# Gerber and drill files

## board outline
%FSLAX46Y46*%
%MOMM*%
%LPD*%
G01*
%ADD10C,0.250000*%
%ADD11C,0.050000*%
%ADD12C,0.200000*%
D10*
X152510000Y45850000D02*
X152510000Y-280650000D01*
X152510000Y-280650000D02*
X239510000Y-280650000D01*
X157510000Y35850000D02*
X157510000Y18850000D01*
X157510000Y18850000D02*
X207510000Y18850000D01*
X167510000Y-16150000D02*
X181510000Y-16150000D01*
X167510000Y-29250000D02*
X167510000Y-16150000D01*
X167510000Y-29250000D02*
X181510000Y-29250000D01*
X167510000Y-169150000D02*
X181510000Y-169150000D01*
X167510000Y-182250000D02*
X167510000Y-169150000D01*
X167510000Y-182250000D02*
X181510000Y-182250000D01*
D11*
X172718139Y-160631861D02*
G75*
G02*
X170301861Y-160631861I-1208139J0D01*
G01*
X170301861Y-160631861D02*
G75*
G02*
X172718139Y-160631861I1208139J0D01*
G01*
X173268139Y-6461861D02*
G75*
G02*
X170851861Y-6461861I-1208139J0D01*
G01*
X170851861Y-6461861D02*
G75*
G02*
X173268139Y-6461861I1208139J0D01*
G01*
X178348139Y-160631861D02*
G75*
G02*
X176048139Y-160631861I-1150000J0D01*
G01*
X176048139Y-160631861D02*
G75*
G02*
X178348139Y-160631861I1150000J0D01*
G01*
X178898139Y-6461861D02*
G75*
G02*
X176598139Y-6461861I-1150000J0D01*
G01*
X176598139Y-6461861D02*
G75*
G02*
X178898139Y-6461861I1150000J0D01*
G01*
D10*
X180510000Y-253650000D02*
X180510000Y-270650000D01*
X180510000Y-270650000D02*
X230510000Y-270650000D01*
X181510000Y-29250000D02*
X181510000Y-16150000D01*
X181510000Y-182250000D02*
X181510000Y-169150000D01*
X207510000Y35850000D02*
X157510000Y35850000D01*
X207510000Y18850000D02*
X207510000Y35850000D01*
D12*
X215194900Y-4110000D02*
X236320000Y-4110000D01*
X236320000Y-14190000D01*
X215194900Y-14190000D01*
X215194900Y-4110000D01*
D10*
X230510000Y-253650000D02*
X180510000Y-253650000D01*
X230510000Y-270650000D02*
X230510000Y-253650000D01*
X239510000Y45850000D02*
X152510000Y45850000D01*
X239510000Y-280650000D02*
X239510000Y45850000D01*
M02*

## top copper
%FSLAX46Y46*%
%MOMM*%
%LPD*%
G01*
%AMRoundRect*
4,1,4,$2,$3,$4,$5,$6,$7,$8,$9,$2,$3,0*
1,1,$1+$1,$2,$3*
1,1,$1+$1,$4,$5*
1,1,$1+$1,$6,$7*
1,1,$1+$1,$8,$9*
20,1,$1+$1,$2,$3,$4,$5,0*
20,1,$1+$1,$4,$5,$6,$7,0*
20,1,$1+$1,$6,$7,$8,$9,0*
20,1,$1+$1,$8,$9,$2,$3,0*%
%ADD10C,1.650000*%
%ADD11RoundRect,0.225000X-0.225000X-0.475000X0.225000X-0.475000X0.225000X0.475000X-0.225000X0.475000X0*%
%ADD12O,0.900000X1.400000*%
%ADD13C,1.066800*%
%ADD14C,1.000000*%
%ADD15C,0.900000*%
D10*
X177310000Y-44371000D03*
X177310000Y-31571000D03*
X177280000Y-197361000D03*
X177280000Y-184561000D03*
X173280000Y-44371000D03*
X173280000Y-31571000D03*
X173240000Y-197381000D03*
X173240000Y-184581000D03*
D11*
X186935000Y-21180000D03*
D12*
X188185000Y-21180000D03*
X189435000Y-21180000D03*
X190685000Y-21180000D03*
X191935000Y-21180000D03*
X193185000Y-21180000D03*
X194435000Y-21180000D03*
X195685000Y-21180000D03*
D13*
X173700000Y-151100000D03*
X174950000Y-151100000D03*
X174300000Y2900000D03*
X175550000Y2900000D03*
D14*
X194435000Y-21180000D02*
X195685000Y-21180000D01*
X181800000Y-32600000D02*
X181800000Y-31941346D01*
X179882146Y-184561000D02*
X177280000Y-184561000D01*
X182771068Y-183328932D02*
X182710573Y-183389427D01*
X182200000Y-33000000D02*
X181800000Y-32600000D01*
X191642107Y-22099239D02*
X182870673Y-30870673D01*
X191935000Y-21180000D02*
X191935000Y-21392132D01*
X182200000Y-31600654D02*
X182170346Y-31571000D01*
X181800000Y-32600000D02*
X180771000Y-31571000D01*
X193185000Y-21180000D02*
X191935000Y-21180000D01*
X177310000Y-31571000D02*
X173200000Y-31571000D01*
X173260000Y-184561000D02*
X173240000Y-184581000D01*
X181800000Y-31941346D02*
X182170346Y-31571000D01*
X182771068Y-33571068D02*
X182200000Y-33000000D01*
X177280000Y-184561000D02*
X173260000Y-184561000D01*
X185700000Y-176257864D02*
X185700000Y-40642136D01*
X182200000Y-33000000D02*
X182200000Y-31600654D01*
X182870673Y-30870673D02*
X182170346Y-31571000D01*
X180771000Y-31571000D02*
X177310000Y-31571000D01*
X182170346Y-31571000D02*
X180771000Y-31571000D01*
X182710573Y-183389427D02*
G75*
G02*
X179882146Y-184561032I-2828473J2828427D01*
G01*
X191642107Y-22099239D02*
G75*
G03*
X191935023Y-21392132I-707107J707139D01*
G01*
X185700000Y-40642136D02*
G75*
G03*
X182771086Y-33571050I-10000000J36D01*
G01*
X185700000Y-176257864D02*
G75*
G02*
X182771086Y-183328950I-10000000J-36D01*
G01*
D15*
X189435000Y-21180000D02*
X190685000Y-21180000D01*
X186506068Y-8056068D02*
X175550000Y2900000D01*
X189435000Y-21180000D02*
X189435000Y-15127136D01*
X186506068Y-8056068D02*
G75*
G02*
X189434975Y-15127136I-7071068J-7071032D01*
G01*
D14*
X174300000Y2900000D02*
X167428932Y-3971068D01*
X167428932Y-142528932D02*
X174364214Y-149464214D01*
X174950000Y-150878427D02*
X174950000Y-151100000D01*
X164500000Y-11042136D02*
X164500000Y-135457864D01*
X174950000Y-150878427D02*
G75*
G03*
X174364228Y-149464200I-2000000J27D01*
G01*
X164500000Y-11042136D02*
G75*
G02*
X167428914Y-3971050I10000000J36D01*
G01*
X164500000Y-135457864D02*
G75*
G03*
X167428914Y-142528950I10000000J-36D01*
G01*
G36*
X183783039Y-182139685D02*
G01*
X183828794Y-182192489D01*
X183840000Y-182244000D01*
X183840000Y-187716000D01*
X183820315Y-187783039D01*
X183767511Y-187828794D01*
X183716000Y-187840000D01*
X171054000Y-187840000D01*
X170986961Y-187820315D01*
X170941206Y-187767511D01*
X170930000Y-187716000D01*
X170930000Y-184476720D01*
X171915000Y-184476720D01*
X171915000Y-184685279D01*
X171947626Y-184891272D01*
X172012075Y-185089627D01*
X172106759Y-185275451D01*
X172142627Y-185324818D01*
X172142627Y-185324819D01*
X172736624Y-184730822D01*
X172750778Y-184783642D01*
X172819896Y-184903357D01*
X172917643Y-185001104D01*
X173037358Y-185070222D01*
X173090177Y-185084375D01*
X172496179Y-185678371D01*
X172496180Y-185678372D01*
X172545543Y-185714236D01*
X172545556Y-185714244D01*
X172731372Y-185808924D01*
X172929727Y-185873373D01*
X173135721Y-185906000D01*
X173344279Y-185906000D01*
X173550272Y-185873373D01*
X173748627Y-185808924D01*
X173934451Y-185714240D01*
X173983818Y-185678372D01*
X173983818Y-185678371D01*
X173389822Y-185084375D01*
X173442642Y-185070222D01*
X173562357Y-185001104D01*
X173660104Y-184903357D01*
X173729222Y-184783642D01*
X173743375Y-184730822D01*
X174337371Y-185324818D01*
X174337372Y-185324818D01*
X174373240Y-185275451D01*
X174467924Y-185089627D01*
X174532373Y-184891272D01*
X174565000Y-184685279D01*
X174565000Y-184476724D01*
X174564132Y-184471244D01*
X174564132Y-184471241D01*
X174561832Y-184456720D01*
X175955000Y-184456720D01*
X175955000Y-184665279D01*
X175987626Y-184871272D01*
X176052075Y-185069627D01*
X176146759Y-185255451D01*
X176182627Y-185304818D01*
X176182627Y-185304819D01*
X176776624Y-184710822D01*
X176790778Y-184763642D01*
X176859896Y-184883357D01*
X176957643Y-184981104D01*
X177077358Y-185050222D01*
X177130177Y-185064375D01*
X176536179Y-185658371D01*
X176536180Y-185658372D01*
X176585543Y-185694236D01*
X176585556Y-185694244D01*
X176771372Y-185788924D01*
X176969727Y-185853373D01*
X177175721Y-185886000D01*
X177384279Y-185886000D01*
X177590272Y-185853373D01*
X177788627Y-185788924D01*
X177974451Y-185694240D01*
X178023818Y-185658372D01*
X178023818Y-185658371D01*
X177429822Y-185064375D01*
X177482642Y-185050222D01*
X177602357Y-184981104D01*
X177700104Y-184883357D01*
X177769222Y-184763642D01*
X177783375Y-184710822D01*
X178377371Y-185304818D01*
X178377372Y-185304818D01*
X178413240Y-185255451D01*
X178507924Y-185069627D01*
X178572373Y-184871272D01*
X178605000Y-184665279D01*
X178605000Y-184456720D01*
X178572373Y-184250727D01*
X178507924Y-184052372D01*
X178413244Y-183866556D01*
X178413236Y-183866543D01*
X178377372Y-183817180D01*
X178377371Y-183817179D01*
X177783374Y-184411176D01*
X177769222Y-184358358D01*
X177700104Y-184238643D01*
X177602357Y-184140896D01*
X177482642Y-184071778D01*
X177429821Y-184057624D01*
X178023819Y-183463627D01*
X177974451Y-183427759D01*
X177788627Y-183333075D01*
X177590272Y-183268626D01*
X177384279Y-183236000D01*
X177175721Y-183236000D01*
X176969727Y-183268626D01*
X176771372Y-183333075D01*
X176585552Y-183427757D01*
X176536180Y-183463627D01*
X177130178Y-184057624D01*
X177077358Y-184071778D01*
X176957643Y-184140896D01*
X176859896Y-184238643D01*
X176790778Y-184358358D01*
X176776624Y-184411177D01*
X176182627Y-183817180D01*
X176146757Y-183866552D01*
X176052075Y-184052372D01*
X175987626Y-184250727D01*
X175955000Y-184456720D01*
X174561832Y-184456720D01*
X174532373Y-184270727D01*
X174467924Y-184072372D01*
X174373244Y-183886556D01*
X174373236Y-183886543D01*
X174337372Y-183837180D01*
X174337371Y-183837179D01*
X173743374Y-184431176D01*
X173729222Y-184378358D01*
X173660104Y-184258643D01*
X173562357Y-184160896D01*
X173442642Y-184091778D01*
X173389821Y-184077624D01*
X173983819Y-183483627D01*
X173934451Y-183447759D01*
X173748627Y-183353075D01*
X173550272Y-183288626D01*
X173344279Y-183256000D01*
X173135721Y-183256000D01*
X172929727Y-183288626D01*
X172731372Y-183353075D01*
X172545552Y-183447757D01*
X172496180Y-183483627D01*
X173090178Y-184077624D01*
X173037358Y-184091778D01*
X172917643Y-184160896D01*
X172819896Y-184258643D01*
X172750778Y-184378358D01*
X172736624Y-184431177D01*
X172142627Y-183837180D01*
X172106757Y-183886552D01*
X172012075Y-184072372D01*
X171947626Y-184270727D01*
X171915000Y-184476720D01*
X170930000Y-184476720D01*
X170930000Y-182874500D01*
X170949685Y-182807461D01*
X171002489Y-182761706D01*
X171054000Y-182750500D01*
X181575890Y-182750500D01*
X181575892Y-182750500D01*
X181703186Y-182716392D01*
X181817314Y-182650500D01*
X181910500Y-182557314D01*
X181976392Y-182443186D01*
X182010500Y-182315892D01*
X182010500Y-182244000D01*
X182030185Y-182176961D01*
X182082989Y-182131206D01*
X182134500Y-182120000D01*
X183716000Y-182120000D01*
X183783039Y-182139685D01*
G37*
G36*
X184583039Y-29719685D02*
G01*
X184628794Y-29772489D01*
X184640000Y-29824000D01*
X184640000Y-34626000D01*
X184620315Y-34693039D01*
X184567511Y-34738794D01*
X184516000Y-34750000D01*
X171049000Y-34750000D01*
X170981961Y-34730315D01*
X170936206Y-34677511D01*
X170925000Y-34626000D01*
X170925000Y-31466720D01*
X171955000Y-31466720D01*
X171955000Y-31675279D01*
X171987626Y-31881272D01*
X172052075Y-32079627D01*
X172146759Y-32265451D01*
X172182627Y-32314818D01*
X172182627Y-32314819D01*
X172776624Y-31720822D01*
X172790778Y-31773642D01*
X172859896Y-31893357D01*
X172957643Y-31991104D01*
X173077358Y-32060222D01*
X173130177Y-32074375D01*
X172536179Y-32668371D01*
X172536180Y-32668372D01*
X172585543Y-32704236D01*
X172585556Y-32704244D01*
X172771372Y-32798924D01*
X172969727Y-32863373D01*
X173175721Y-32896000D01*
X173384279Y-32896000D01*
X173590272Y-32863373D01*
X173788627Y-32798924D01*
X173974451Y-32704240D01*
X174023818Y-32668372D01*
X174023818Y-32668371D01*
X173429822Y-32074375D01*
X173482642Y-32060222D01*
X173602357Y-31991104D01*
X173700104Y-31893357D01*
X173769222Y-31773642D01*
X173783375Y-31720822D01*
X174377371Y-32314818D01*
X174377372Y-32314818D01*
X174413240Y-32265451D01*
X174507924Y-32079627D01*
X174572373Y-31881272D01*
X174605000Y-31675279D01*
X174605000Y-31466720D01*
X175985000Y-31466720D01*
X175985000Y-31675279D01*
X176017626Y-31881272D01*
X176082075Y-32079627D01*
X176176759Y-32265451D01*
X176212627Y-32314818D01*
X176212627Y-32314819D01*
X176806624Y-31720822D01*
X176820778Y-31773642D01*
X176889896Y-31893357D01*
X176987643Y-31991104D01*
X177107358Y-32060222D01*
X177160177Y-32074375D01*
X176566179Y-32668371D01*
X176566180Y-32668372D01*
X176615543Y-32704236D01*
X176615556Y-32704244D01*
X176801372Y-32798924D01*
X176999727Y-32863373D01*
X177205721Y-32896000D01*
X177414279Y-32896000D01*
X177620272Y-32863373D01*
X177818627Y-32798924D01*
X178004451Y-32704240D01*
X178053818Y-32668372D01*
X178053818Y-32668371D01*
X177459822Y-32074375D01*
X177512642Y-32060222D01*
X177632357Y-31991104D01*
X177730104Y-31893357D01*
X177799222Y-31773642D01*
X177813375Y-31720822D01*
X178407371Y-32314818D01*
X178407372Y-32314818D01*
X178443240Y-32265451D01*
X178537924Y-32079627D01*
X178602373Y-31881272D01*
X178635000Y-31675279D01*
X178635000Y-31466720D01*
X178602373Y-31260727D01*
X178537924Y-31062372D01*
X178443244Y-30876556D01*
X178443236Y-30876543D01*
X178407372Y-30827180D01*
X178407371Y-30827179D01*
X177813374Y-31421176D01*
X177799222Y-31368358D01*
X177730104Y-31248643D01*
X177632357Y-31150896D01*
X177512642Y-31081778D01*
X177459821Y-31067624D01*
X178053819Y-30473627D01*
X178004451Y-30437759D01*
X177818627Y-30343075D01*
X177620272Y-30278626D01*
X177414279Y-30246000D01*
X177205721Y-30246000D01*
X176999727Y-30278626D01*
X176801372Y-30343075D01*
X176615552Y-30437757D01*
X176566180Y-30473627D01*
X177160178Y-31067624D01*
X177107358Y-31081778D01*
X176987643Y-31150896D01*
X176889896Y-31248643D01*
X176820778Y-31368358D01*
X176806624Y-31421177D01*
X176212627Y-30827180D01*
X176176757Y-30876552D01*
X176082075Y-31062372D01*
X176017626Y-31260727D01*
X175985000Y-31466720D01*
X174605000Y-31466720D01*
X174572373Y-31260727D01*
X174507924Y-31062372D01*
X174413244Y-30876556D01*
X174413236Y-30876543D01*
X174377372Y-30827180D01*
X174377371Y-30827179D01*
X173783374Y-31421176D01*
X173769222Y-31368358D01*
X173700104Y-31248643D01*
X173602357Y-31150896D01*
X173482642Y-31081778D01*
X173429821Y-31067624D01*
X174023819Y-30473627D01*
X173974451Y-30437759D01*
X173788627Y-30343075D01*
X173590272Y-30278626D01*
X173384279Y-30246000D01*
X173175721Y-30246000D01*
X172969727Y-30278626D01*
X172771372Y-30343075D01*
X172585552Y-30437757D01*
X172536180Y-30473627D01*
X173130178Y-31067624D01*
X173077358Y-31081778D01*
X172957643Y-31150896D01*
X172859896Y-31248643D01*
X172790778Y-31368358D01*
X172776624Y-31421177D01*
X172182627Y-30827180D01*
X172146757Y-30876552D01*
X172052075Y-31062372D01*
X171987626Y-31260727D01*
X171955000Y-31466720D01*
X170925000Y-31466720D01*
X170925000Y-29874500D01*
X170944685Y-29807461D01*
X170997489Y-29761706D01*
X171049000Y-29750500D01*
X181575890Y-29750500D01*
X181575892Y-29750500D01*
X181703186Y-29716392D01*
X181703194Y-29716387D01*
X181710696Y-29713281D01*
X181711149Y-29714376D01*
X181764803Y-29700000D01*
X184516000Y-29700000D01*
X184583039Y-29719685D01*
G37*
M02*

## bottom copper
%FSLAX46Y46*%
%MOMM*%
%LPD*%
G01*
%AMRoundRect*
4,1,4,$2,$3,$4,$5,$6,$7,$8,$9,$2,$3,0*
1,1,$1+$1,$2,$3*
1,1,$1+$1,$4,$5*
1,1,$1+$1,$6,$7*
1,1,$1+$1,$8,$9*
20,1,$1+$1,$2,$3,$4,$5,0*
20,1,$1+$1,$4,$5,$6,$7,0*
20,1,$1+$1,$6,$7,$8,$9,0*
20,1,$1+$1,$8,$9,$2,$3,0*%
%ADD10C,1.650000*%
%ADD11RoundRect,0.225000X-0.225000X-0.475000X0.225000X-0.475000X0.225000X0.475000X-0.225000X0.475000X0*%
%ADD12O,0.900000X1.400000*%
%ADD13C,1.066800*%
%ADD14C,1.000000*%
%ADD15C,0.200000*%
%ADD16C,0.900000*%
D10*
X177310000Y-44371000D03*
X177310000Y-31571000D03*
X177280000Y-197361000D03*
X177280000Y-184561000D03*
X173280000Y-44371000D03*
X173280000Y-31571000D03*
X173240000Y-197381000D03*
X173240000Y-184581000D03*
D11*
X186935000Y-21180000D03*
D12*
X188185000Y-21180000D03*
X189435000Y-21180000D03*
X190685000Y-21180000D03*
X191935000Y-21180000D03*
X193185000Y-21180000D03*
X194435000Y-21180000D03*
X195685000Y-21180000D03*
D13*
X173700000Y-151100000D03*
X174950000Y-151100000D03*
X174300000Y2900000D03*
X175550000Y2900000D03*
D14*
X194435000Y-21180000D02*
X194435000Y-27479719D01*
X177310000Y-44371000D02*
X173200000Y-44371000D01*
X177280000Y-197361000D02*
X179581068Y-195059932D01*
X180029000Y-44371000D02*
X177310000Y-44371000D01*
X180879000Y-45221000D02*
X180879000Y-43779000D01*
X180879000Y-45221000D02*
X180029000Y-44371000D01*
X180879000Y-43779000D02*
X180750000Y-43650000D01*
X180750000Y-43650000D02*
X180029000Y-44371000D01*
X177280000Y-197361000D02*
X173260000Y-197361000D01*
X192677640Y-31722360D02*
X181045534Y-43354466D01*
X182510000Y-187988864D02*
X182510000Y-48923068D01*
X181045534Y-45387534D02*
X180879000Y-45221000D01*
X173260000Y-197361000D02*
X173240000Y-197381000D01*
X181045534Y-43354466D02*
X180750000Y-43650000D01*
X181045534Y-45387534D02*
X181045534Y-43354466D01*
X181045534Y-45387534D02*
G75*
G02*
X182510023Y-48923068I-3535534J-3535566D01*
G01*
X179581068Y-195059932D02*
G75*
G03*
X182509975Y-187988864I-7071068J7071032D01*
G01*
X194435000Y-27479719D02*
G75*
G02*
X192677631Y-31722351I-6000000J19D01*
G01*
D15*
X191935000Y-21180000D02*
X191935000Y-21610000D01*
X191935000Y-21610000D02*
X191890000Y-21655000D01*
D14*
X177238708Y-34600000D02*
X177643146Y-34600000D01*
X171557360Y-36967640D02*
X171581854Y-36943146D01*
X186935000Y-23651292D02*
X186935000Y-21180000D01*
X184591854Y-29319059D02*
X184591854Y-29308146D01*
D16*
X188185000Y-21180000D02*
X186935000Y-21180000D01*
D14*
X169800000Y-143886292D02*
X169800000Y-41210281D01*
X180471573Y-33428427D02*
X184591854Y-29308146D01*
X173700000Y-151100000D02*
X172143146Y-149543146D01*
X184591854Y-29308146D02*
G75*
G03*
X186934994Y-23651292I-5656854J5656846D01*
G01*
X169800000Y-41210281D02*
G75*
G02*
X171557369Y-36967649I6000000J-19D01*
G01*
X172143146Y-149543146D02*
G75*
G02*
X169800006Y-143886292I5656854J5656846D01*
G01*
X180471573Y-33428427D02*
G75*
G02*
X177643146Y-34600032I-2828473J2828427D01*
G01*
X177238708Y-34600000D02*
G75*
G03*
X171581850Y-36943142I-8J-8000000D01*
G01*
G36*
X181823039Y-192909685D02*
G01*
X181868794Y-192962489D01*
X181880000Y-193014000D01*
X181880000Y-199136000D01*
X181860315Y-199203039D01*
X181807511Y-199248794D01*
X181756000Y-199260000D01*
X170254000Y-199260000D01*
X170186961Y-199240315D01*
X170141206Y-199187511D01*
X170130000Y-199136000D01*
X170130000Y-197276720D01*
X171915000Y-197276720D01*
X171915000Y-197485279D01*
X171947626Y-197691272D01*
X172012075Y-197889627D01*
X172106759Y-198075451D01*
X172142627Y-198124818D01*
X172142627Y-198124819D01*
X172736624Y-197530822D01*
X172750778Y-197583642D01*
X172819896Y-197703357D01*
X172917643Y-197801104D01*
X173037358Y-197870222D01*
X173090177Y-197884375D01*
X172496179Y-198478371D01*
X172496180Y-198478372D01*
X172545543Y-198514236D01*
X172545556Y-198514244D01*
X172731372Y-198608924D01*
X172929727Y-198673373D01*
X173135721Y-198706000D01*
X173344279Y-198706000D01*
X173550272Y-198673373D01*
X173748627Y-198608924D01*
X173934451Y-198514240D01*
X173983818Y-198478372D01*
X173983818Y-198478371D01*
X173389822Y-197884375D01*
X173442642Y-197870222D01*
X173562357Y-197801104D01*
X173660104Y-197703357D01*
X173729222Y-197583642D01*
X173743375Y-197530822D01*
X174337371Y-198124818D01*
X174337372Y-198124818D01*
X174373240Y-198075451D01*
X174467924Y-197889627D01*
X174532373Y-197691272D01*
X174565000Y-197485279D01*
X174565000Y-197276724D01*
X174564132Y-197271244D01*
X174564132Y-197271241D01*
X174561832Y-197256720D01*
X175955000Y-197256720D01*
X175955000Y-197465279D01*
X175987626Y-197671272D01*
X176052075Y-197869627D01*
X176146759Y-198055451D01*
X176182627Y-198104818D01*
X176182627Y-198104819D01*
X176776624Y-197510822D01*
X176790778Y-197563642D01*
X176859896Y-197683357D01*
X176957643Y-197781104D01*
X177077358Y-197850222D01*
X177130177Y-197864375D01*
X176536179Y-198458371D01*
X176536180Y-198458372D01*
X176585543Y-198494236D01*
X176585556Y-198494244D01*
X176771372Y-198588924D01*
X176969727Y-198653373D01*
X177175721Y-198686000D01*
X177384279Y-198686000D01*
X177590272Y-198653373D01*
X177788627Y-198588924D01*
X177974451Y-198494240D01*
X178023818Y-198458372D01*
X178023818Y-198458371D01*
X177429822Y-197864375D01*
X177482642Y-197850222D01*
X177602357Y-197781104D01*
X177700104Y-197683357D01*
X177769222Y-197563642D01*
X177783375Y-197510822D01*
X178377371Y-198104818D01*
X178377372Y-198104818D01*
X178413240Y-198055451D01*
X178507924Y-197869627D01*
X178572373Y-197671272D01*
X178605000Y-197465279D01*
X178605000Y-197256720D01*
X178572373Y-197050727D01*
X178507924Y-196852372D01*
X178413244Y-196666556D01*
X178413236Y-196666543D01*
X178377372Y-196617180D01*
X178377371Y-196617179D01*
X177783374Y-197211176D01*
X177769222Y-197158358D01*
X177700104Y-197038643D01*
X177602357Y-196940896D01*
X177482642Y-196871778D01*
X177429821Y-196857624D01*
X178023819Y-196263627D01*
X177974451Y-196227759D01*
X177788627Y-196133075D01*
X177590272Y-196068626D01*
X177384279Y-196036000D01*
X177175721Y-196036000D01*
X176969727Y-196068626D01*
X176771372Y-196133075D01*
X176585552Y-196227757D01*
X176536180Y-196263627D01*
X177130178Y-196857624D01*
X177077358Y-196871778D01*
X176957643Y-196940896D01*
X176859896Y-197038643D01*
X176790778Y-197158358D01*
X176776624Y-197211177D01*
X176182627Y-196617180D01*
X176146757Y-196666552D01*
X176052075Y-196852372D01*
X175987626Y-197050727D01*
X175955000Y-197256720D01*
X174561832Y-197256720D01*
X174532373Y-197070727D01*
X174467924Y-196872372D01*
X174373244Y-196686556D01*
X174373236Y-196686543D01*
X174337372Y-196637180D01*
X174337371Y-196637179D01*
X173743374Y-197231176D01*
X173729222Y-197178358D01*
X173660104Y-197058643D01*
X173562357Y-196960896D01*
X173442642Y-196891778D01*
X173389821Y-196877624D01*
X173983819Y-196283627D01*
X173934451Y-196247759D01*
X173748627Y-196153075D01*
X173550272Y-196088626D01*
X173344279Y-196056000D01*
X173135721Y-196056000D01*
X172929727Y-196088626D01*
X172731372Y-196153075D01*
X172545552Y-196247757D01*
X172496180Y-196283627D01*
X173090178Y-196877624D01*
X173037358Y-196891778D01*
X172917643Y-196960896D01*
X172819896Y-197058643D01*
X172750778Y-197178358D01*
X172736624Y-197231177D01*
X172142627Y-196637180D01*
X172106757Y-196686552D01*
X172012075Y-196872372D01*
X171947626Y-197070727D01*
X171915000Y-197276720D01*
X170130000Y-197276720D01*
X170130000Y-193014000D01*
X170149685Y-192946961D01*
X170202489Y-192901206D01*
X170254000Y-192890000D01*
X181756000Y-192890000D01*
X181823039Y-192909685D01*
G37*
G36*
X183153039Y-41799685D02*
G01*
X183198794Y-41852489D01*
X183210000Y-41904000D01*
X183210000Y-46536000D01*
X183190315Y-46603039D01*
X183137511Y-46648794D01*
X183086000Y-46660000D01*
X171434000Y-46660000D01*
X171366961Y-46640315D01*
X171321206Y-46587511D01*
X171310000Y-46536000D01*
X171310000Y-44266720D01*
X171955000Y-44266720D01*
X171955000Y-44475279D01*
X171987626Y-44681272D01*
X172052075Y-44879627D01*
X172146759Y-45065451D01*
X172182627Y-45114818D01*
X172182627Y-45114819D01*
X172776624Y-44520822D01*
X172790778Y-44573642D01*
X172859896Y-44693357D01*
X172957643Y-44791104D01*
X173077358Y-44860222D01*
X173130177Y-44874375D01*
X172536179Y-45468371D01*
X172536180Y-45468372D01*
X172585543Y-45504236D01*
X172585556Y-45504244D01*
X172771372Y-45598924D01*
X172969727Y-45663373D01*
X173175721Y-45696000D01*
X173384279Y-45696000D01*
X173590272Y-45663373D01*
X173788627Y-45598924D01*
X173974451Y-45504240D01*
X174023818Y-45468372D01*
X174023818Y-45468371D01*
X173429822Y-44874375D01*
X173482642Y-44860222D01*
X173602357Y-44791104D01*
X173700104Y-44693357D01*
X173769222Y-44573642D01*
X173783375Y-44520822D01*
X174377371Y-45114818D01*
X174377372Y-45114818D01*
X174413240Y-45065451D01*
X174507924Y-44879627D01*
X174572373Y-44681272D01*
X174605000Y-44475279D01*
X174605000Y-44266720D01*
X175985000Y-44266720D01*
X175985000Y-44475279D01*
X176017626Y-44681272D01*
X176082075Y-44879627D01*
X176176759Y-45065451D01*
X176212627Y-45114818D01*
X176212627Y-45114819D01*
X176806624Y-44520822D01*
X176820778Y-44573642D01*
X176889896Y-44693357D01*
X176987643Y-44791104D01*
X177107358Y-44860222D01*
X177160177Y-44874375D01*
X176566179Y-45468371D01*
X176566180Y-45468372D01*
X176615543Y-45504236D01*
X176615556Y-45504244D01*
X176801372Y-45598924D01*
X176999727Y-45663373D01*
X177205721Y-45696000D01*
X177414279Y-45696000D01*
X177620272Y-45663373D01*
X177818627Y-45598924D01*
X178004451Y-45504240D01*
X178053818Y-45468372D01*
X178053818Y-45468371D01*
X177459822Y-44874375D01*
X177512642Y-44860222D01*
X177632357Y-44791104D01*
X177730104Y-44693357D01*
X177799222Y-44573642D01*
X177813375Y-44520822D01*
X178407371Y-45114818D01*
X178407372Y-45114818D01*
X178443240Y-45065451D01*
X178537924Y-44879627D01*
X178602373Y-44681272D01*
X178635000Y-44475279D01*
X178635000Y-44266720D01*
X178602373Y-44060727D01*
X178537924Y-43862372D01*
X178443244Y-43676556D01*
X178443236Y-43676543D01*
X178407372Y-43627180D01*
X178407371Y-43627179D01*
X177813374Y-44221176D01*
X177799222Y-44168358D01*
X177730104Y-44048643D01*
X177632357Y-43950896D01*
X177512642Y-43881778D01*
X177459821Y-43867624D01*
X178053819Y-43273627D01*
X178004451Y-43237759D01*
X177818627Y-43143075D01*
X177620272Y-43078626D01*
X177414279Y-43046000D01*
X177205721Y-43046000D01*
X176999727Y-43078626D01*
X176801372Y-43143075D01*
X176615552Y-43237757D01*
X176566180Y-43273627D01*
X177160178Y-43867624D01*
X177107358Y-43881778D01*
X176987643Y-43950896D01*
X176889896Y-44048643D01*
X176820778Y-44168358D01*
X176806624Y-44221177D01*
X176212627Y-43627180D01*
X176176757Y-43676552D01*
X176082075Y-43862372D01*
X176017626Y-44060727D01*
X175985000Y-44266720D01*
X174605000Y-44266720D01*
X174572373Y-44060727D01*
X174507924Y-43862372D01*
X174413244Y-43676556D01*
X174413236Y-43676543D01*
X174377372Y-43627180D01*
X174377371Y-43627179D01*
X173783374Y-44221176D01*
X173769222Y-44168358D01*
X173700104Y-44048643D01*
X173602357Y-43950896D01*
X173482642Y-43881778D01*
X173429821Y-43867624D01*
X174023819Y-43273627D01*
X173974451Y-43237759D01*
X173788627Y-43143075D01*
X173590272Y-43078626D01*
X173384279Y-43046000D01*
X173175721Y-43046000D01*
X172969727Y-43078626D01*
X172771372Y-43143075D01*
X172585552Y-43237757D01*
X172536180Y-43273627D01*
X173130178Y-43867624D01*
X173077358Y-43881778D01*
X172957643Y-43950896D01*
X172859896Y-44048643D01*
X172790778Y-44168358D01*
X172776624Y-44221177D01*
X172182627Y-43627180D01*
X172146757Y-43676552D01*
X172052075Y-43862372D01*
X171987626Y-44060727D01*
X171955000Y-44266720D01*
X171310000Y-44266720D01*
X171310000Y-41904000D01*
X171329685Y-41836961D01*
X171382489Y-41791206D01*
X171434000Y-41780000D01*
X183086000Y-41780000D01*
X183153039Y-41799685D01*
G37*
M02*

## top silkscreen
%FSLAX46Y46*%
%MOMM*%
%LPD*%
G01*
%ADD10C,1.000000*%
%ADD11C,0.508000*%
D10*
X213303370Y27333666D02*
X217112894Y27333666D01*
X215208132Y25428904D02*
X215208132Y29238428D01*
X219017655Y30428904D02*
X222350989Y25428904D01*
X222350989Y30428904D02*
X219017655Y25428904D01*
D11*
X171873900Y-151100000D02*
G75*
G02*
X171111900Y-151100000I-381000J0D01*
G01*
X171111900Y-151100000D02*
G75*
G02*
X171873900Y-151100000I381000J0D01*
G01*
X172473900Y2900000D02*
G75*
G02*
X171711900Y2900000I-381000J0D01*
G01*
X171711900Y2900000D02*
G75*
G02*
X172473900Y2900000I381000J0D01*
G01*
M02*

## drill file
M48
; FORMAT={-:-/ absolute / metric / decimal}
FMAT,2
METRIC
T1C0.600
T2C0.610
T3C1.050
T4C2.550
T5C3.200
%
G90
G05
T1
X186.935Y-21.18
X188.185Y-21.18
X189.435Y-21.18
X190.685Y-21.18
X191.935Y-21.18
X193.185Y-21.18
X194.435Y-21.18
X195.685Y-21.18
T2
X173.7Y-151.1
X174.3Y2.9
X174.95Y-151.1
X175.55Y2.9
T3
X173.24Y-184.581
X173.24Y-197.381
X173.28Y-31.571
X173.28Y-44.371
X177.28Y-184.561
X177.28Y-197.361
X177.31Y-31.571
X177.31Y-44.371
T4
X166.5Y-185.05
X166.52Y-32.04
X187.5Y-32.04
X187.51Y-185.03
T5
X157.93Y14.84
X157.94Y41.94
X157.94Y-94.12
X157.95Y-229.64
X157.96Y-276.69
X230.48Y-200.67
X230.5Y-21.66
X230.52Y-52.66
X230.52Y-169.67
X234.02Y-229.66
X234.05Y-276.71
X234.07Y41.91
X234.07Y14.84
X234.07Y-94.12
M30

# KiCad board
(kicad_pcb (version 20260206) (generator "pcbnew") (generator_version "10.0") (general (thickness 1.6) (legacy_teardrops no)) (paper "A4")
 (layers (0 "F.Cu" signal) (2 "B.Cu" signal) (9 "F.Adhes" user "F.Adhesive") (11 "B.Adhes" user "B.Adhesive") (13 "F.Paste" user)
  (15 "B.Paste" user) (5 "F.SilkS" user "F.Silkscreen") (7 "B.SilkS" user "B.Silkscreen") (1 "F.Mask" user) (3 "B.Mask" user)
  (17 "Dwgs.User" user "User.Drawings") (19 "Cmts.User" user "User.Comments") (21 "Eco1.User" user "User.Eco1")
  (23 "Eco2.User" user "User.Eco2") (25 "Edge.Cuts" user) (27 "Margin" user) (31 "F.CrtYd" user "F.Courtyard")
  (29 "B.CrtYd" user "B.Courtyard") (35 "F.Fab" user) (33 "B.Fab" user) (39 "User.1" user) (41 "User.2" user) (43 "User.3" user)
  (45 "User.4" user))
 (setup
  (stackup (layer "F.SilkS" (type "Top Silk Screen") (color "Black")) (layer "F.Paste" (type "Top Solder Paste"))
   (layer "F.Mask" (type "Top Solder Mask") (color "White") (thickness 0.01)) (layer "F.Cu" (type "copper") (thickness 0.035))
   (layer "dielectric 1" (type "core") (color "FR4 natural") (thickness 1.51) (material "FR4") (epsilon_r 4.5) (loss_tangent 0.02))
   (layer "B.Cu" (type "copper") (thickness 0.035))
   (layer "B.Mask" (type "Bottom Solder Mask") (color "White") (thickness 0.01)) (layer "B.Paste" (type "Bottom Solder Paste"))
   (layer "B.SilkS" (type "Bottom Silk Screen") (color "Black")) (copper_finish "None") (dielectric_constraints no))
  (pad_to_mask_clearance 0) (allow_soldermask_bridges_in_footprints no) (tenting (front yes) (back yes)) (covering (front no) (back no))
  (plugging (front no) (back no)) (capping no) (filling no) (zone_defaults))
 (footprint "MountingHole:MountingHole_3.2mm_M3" (layer "F.Cu") (at 230.52 169.67 180)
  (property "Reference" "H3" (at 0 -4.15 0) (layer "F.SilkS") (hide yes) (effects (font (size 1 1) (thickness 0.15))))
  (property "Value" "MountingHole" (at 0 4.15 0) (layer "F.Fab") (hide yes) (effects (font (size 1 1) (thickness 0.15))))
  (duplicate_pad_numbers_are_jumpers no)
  (pad "" np_thru_hole circle (at 0 0 180) (size 3.2 3.2) (drill 3.2) (layers "*.Cu" "*.Mask")))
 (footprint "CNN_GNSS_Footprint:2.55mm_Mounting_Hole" (layer "F.Cu") (at 187.5 32.12)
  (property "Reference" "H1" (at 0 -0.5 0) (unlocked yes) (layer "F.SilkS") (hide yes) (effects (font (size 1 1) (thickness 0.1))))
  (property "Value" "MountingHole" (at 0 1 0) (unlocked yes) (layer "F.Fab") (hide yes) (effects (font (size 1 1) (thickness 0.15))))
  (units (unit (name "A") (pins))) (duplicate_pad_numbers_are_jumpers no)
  (pad "" np_thru_hole circle (at 0 -0.08) (size 2.55 2.55) (drill 2.55) (layers "*.Cu" "*.Mask")))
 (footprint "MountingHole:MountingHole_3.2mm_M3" (layer "F.Cu") (at 234.07 -41.91 180)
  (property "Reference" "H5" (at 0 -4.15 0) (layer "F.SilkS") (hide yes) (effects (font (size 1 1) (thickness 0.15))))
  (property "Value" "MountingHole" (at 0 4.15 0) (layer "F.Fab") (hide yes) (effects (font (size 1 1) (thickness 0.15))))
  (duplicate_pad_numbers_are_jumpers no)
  (pad "" np_thru_hole circle (at 0 0 180) (size 3.2 3.2) (drill 3.2) (layers "*.Cu" "*.Mask")))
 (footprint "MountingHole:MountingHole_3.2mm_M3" (layer "F.Cu") (at 230.48 200.67 180)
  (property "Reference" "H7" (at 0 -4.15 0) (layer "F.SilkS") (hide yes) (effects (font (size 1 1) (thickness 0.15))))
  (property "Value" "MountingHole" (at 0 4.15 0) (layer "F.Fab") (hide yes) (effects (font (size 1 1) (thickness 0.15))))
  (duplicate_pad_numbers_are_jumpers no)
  (pad "" np_thru_hole circle (at 0 0 180) (size 3.2 3.2) (drill 3.2) (layers "*.Cu" "*.Mask")))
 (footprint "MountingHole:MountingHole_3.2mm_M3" (layer "F.Cu") (at 157.94 -41.94 180)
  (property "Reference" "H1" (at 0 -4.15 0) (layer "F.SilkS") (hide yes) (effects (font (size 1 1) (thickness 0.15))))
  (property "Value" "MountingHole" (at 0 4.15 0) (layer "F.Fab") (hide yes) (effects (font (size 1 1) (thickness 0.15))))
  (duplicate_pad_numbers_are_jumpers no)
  (pad "" np_thru_hole circle (at 0 0 180) (size 3.2 3.2) (drill 3.2) (layers "*.Cu" "*.Mask")))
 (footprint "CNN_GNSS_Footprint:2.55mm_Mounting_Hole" (layer "F.Cu") (at 166.5 185.13)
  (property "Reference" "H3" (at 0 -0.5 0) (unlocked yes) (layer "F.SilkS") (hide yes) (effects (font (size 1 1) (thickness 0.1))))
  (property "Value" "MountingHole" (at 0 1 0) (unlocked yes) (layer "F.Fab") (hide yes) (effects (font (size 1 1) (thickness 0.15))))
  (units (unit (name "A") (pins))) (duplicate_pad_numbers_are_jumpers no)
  (pad "" np_thru_hole circle (at 0 -0.08) (size 2.55 2.55) (drill 2.55) (layers "*.Cu" "*.Mask")))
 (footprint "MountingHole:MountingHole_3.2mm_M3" (layer "F.Cu") (at 234.05 276.71 180)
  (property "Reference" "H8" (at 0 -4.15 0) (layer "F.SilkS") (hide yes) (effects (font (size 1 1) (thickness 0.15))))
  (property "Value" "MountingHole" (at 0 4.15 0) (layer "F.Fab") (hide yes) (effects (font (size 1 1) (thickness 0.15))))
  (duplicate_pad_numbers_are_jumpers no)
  (pad "" np_thru_hole circle (at 0 0 180) (size 3.2 3.2) (drill 3.2) (layers "*.Cu" "*.Mask")))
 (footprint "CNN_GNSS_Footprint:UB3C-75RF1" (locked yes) (layer "F.Cu") (at 177.31 44.371 90)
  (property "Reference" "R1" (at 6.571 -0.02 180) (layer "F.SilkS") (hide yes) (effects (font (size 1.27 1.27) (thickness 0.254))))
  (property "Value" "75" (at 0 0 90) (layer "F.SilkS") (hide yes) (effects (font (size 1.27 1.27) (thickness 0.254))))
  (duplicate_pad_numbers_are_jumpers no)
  (pad "1" thru_hole circle (at 0 0 90) (size 1.65 1.65) (drill 1.05) (layers "*.Cu" "*.Mask") (remove_unused_layers no) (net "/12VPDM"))
  (pad "2" thru_hole circle (at 12.8 0 90) (size 1.65 1.65) (drill 1.05) (layers "*.Cu" "*.Mask") (remove_unused_layers no)
   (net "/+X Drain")))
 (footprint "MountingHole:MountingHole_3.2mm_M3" (layer "F.Cu") (at 230.52 52.66 180)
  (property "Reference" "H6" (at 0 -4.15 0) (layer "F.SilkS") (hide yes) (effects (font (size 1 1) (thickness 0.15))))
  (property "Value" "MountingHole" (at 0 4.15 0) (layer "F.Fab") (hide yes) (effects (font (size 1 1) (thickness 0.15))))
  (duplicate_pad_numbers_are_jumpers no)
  (pad "" np_thru_hole circle (at 0 0 180) (size 3.2 3.2) (drill 3.2) (layers "*.Cu" "*.Mask")))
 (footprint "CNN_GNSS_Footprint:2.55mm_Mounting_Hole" (layer "F.Cu") (at 166.52 32.12)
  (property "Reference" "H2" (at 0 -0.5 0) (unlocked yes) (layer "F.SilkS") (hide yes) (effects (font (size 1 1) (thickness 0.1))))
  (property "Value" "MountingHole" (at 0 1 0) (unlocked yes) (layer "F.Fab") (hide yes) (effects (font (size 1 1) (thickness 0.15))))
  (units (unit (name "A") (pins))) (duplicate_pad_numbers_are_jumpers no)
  (pad "" np_thru_hole circle (at 0 -0.08) (size 2.55 2.55) (drill 2.55) (layers "*.Cu" "*.Mask")))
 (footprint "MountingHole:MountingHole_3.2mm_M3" (layer "F.Cu") (at 234.07 -14.84 180)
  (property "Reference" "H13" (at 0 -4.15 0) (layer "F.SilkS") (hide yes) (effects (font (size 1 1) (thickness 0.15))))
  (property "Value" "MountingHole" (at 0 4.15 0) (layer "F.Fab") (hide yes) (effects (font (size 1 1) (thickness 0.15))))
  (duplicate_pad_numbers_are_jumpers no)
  (pad "" np_thru_hole circle (at 0 0 180) (size 3.2 3.2) (drill 3.2) (layers "*.Cu" "*.Mask")))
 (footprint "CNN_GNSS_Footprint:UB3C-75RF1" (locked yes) (layer "F.Cu") (at 177.28 197.361 90)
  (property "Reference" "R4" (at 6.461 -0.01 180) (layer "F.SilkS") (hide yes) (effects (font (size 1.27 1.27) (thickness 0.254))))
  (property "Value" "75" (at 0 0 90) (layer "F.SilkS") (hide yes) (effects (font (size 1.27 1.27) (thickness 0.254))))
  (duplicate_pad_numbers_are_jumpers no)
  (pad "1" thru_hole circle (at 0 0 90) (size 1.65 1.65) (drill 1.05) (layers "*.Cu" "*.Mask") (remove_unused_layers no) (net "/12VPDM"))
  (pad "2" thru_hole circle (at 12.8 0 90) (size 1.65 1.65) (drill 1.05) (layers "*.Cu" "*.Mask") (remove_unused_layers no)
   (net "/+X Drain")))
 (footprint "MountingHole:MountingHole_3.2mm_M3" (layer "F.Cu") (at 234.07 94.12 180)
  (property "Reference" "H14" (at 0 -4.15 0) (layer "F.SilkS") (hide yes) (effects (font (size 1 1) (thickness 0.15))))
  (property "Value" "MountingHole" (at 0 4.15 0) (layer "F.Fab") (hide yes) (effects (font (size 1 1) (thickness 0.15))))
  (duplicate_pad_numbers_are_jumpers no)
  (pad "" np_thru_hole circle (at 0 0 180) (size 3.2 3.2) (drill 3.2) (layers "*.Cu" "*.Mask")))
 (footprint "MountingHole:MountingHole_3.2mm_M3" (layer "F.Cu") (at 157.94 94.12 180)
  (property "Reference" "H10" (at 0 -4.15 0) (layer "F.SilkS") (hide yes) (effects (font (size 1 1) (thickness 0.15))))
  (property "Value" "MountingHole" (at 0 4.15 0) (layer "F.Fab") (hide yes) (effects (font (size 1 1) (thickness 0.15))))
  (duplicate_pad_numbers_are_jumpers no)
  (pad "" np_thru_hole circle (at 0 0 180) (size 3.2 3.2) (drill 3.2) (layers "*.Cu" "*.Mask")))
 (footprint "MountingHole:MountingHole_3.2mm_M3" (layer "F.Cu") (at 230.5 21.66 180)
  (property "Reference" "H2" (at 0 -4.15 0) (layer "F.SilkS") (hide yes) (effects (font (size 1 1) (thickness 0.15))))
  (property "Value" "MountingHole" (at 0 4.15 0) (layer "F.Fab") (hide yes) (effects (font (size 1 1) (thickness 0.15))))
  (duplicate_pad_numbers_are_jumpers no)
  (pad "" np_thru_hole circle (at 0 0 180) (size 3.2 3.2) (drill 3.2) (layers "*.Cu" "*.Mask")))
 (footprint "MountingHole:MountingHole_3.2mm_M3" (layer "F.Cu") (at 234.02 229.66 180)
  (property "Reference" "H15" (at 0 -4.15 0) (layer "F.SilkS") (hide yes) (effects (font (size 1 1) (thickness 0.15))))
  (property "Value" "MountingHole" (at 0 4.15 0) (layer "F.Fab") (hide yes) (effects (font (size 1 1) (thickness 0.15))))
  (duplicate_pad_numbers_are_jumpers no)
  (pad "" np_thru_hole circle (at 0 0 180) (size 3.2 3.2) (drill 3.2) (layers "*.Cu" "*.Mask")))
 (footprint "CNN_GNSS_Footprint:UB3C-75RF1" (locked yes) (layer "F.Cu") (at 173.28 44.371 90)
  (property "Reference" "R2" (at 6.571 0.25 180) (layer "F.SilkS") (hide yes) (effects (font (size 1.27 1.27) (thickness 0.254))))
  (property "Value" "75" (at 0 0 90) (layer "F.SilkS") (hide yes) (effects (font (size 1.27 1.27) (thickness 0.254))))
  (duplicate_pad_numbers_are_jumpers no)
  (pad "1" thru_hole circle (at 0 0 90) (size 1.65 1.65) (drill 1.05) (layers "*.Cu" "*.Mask") (remove_unused_layers no) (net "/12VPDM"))
  (pad "2" thru_hole circle (at 12.8 0 90) (size 1.65 1.65) (drill 1.05) (layers "*.Cu" "*.Mask") (remove_unused_layers no)
   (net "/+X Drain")))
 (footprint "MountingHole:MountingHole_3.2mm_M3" (layer "F.Cu") (at 157.95 229.64 180)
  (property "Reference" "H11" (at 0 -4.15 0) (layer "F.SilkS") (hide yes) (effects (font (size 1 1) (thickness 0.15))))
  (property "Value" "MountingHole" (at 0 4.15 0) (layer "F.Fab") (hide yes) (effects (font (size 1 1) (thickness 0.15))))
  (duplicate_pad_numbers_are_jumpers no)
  (pad "" np_thru_hole circle (at 0 0 180) (size 3.2 3.2) (drill 3.2) (layers "*.Cu" "*.Mask")))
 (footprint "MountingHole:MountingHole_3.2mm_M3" (layer "F.Cu") (at 157.93 -14.84 180)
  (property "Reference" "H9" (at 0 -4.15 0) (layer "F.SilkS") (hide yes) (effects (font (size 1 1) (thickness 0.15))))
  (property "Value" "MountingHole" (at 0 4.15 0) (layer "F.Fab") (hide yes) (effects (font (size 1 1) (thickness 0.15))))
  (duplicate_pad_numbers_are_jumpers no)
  (pad "" np_thru_hole circle (at 0 0 180) (size 3.2 3.2) (drill 3.2) (layers "*.Cu" "*.Mask")))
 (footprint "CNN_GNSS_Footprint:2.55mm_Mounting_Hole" (layer "F.Cu") (at 187.51 185.11)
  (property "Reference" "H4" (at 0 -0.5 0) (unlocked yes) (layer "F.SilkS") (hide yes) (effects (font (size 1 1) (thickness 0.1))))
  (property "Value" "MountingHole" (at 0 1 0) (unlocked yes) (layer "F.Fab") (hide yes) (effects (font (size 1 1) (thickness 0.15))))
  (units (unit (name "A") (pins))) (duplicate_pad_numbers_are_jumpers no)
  (pad "" np_thru_hole circle (at 0 -0.08) (size 2.55 2.55) (drill 2.55) (layers "*.Cu" "*.Mask")))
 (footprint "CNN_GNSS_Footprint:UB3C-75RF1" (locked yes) (layer "F.Cu") (at 173.24 197.381 90)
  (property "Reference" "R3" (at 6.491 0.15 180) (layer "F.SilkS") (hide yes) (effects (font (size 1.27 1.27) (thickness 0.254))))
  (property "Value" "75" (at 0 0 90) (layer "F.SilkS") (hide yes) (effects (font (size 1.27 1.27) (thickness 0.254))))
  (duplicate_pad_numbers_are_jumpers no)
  (pad "1" thru_hole circle (at 0 0 90) (size 1.65 1.65) (drill 1.05) (layers "*.Cu" "*.Mask") (remove_unused_layers no) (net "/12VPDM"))
  (pad "2" thru_hole circle (at 12.8 0 90) (size 1.65 1.65) (drill 1.05) (layers "*.Cu" "*.Mask") (remove_unused_layers no)
   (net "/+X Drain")))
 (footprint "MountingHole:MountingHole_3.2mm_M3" (layer "F.Cu") (at 157.96 276.69 180)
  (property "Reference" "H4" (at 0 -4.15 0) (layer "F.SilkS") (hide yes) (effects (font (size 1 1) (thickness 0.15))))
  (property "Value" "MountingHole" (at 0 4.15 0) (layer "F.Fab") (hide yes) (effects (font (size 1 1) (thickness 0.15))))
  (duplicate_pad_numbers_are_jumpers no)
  (pad "" np_thru_hole circle (at 0 0 180) (size 3.2 3.2) (drill 3.2) (layers "*.Cu" "*.Mask")))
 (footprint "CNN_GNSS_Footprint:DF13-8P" (layer "B.Cu") (at 190.98 21.73)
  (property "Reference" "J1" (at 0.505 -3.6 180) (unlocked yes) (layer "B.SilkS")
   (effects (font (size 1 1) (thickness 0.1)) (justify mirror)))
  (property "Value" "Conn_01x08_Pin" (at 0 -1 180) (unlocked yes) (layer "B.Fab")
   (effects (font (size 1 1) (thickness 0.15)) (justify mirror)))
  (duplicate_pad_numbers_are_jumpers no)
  (pad "1" thru_hole roundrect (at -4.045 -0.55) (size 0.9 1.4) (drill 0.6) (layers "*.Cu" "*.Mask") (remove_unused_layers no)
   (roundrect_rratio 0.25) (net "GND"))
  (pad "2" thru_hole oval (at -2.795 -0.55) (size 0.9 1.4) (drill 0.6) (layers "*.Cu" "*.Mask") (remove_unused_layers no) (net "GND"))
  (pad "3" thru_hole oval (at -1.545 -0.55) (size 0.9 1.4) (drill 0.6) (layers "*.Cu" "*.Mask") (remove_unused_layers no)
   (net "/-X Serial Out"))
  (pad "4" thru_hole oval (at -0.295 -0.55) (size 0.9 1.4) (drill 0.6) (layers "*.Cu" "*.Mask") (remove_unused_layers no)
   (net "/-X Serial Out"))
  (pad "5" thru_hole oval (at 0.955 -0.55) (size 0.9 1.4) (drill 0.6) (layers "*.Cu" "*.Mask") (remove_unused_layers no) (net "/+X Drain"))
  (pad "6" thru_hole oval (at 2.205 -0.55) (size 0.9 1.4) (drill 0.6) (layers "*.Cu" "*.Mask") (remove_unused_layers no) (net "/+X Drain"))
  (pad "7" thru_hole oval (at 3.455 -0.55) (size 0.9 1.4) (drill 0.6) (layers "*.Cu" "*.Mask") (remove_unused_layers no) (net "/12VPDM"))
  (pad "8" thru_hole oval (at 4.705 -0.55) (size 0.9 1.4) (drill 0.6) (layers "*.Cu" "*.Mask") (remove_unused_layers no) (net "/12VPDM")))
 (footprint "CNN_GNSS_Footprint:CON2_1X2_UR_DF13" (layer "B.Cu") (at 173.7 151.1 180)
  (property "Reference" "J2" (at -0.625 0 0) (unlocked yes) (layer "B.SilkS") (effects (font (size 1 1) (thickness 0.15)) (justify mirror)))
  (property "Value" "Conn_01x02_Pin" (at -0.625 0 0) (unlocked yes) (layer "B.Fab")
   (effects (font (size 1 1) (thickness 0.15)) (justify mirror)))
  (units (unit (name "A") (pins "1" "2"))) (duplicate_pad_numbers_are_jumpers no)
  (fp_circle (center 2.2071 0) (end 2.5881 0) (stroke (width 0.508) (type solid)) (fill no) (layer "F.SilkS"))
  (pad "1" thru_hole circle (at 0 0 180) (size 1.0668 1.0668) (drill 0.6096) (layers "*.Cu" "*.Mask") (remove_unused_layers no) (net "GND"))
  (pad "2" thru_hole circle (at -1.25 0 180) (size 1.0668 1.0668) (drill 0.6096) (layers "*.Cu" "*.Mask") (remove_unused_layers no)
   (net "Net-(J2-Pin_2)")))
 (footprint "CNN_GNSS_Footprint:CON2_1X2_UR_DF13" (layer "B.Cu") (at 174.3 -2.9 180)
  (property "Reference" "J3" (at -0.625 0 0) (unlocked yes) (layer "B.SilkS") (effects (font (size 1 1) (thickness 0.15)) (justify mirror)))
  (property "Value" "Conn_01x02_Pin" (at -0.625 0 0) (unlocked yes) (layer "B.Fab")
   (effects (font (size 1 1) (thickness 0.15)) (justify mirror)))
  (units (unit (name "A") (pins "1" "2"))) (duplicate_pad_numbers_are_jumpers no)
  (fp_circle (center 2.2071 0) (end 2.5881 0) (stroke (width 0.508) (type solid)) (fill no) (layer "F.SilkS"))
  (pad "1" thru_hole circle (at 0 0 180) (size 1.0668 1.0668) (drill 0.6096) (layers "*.Cu" "*.Mask") (remove_unused_layers no)
   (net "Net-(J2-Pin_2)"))
  (pad "2" thru_hole circle (at -1.25 0 180) (size 1.0668 1.0668) (drill 0.6096) (layers "*.Cu" "*.Mask") (remove_unused_layers no)
   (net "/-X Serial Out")))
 (gr_line (start 152.51 -45.85) (end 152.51 280.65) (stroke (width 0.25) (type default)) (layer "Edge.Cuts"))
 (gr_line (start 152.51 280.65) (end 239.51 280.65) (stroke (width 0.25) (type default)) (layer "Edge.Cuts"))
 (gr_line (start 157.51 -35.85) (end 157.51 -18.85) (stroke (width 0.25) (type default)) (layer "Edge.Cuts"))
 (gr_line (start 157.51 -18.85) (end 207.51 -18.85) (stroke (width 0.25) (type default)) (layer "Edge.Cuts"))
 (gr_line (start 167.51 16.15) (end 181.51 16.15) (stroke (width 0.25) (type default)) (layer "Edge.Cuts"))
 (gr_line (start 167.51 29.25) (end 167.51 16.15) (stroke (width 0.25) (type default)) (layer "Edge.Cuts"))
 (gr_line (start 167.51 29.25) (end 181.51 29.25) (stroke (width 0.25) (type default)) (layer "Edge.Cuts"))
 (gr_line (start 167.51 169.15) (end 181.51 169.15) (stroke (width 0.25) (type default)) (layer "Edge.Cuts"))
 (gr_line (start 167.51 182.25) (end 167.51 169.15) (stroke (width 0.25) (type default)) (layer "Edge.Cuts"))
 (gr_line (start 167.51 182.25) (end 181.51 182.25) (stroke (width 0.25) (type default)) (layer "Edge.Cuts"))
 (gr_circle (center 171.51 160.631861) (end 171.91 161.771861) (stroke (width 0.05) (type default)) (fill no) (layer "Edge.Cuts"))
 (gr_circle (center 172.06 6.461861) (end 172.46 7.601861) (stroke (width 0.05) (type default)) (fill no) (layer "Edge.Cuts"))
 (gr_circle (center 177.198139 160.631861) (end 178.348139 160.631861) (stroke (width 0.05) (type solid)) (fill no) (layer "Edge.Cuts"))
 (gr_circle (center 177.748139 6.461861) (end 178.898139 6.461861) (stroke (width 0.05) (type solid)) (fill no) (layer "Edge.Cuts"))
 (gr_line (start 180.51 253.65) (end 180.51 270.65) (stroke (width 0.25) (type default)) (layer "Edge.Cuts"))
 (gr_line (start 180.51 270.65) (end 230.51 270.65) (stroke (width 0.25) (type default)) (layer "Edge.Cuts"))
 (gr_line (start 181.51 29.25) (end 181.51 16.15) (stroke (width 0.25) (type default)) (layer "Edge.Cuts"))
 (gr_line (start 181.51 182.25) (end 181.51 169.15) (stroke (width 0.25) (type default)) (layer "Edge.Cuts"))
 (gr_line (start 207.51 -35.85) (end 157.51 -35.85) (stroke (width 0.25) (type default)) (layer "Edge.Cuts"))
 (gr_line (start 207.51 -18.85) (end 207.51 -35.85) (stroke (width 0.25) (type default)) (layer "Edge.Cuts"))
 (gr_rect (start 215.1949 4.11) (end 236.32 14.19) (stroke (width 0.2) (type solid)) (fill no) (layer "Edge.Cuts"))
 (gr_line (start 230.51 253.65) (end 180.51 253.65) (stroke (width 0.25) (type default)) (layer "Edge.Cuts"))
 (gr_line (start 230.51 270.65) (end 230.51 253.65) (stroke (width 0.25) (type default)) (layer "Edge.Cuts"))
 (gr_line (start 239.51 -45.85) (end 152.51 -45.85) (stroke (width 0.25) (type default)) (layer "Edge.Cuts"))
 (gr_line (start 239.51 280.65) (end 239.51 -45.85) (stroke (width 0.25) (type default)) (layer "Edge.Cuts"))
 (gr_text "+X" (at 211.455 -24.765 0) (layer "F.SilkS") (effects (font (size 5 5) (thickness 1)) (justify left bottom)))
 (segment (start 194.435 21.18) (end 195.685 21.18) (width 1) (layer "F.Cu") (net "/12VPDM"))
 (segment (start 194.435 21.18) (end 194.435 27.479719) (width 1) (layer "B.Cu") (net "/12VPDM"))
 (segment (start 177.31 44.371) (end 173.2 44.371) (width 1) (layer "B.Cu") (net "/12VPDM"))
 (segment (start 177.28 197.361) (end 179.581068 195.059932) (width 1) (layer "B.Cu") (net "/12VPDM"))
 (segment (start 180.029 44.371) (end 177.31 44.371) (width 1) (layer "B.Cu") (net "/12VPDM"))
 (segment (start 180.879 45.221) (end 180.879 43.779) (width 1) (layer "B.Cu") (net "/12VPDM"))
 (segment (start 180.879 45.221) (end 180.029 44.371) (width 1) (layer "B.Cu") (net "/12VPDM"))
 (segment (start 180.879 43.779) (end 180.75 43.65) (width 1) (layer "B.Cu") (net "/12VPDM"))
 (segment (start 180.75 43.65) (end 180.029 44.371) (width 1) (layer "B.Cu") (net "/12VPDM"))
 (segment (start 177.28 197.361) (end 173.26 197.361) (width 1) (layer "B.Cu") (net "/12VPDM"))
 (segment (start 192.67764 31.72236) (end 181.045534 43.354466) (width 1) (layer "B.Cu") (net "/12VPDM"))
 (segment (start 182.51 187.988864) (end 182.51 48.923068) (width 1) (layer "B.Cu") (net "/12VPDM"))
 (segment (start 181.045534 45.387534) (end 180.879 45.221) (width 1) (layer "B.Cu") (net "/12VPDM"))
 (segment (start 173.26 197.361) (end 173.24 197.381) (width 1) (layer "B.Cu") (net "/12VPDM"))
 (segment (start 181.045534 43.354466) (end 180.75 43.65) (width 1) (layer "B.Cu") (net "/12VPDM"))
 (segment (start 181.045534 45.387534) (end 181.045534 43.354466) (width 1) (layer "B.Cu") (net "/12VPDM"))
 (arc (start 181.045534 45.387534) (mid 182.129398 47.009651) (end 182.51 48.923068) (width 1) (layer "B.Cu") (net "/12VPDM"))
 (arc (start 179.581068 195.059932) (mid 181.748796 191.815698) (end 182.51 187.988864) (width 1) (layer "B.Cu") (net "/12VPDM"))
 (arc (start 194.435 27.479719) (mid 193.978277 29.77582) (end 192.67764 31.72236) (width 1) (layer "B.Cu") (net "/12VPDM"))
 (segment (start 181.8 32.6) (end 181.8 31.941346) (width 1) (layer "F.Cu") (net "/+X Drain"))
 (segment (start 179.882146 184.561) (end 177.28 184.561) (width 1) (layer "F.Cu") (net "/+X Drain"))
 (segment (start 182.771068 183.328932) (end 182.710573 183.389427) (width 1) (layer "F.Cu") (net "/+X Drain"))
 (segment (start 182.2 33) (end 181.8 32.6) (width 1) (layer "F.Cu") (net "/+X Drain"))
 (segment (start 191.642107 22.099239) (end 182.870673 30.870673) (width 1) (layer "F.Cu") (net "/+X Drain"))
 (segment (start 191.935 21.18) (end 191.935 21.392132) (width 1) (layer "F.Cu") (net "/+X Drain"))
 (segment (start 182.2 31.600654) (end 182.170346 31.571) (width 1) (layer "F.Cu") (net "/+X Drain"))
 (segment (start 181.8 32.6) (end 180.771 31.571) (width 1) (layer "F.Cu") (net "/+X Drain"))
 (segment (start 193.185 21.18) (end 191.935 21.18) (width 1) (layer "F.Cu") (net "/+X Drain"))
 (segment (start 177.31 31.571) (end 173.2 31.571) (width 1) (layer "F.Cu") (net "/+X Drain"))
 (segment (start 173.26 184.561) (end 173.24 184.581) (width 1) (layer "F.Cu") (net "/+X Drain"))
 (segment (start 181.8 31.941346) (end 182.170346 31.571) (width 1) (layer "F.Cu") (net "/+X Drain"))
 (segment (start 182.771068 33.571068) (end 182.2 33) (width 1) (layer "F.Cu") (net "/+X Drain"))
 (segment (start 177.28 184.561) (end 173.26 184.561) (width 1) (layer "F.Cu") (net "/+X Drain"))
 (segment (start 185.7 176.257864) (end 185.7 40.642136) (width 1) (layer "F.Cu") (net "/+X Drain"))
 (segment (start 182.2 33) (end 182.2 31.600654) (width 1) (layer "F.Cu") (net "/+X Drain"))
 (segment (start 182.870673 30.870673) (end 182.170346 31.571) (width 1) (layer "F.Cu") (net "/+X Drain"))
 (segment (start 180.771 31.571) (end 177.31 31.571) (width 1) (layer "F.Cu") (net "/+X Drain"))
 (segment (start 182.170346 31.571) (end 180.771 31.571) (width 1) (layer "F.Cu") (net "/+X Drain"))
 (arc (start 182.710573 183.389427) (mid 181.41288 184.256518) (end 179.882146 184.561) (width 1) (layer "F.Cu") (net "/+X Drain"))
 (arc (start 191.642107 22.099239) (mid 191.85888 21.774816) (end 191.935 21.392132) (width 1) (layer "F.Cu") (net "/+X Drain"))
 (arc (start 185.7 40.642136) (mid 184.938795 36.815302) (end 182.771068 33.571068) (width 1) (layer "F.Cu") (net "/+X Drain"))
 (arc (start 185.7 176.257864) (mid 184.938795 180.084698) (end 182.771068 183.328932) (width 1) (layer "F.Cu") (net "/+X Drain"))
 (segment (start 191.935 21.18) (end 191.935 21.61) (width 0.2) (layer "B.Cu") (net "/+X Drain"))
 (segment (start 191.935 21.61) (end 191.89 21.655) (width 0.2) (layer "B.Cu") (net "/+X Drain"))
 (segment (start 177.238708 34.6) (end 177.643146 34.6) (width 1) (layer "B.Cu") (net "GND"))
 (segment (start 171.55736 36.96764) (end 171.581854 36.943146) (width 1) (layer "B.Cu") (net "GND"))
 (segment (start 186.935 23.651292) (end 186.935 21.18) (width 1) (layer "B.Cu") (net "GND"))
 (segment (start 184.591854 29.319059) (end 184.591854 29.308146) (width 1) (layer "B.Cu") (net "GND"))
 (segment (start 188.185 21.18) (end 186.935 21.18) (width 0.9) (layer "B.Cu") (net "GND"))
 (segment (start 169.8 143.886292) (end 169.8 41.210281) (width 1) (layer "B.Cu") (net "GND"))
 (segment (start 180.471573 33.428427) (end 184.591854 29.308146) (width 1) (layer "B.Cu") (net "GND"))
 (segment (start 173.7 151.1) (end 172.143146 149.543146) (width 1) (layer "B.Cu") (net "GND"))
 (arc (start 184.591854 29.308146) (mid 186.326036 26.712759) (end 186.935 23.651292) (width 1) (layer "B.Cu") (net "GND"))
 (arc (start 169.8 41.210281) (mid 170.256723 38.91418) (end 171.55736 36.96764) (width 1) (layer "B.Cu") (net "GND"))
 (arc (start 172.143146 149.543146) (mid 170.408964 146.947759) (end 169.8 143.886292) (width 1) (layer "B.Cu") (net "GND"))
 (arc (start 180.471573 33.428427) (mid 179.17388 34.295518) (end 177.643146 34.6) (width 1) (layer "B.Cu") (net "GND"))
 (arc (start 177.238708 34.6) (mid 174.177241 35.208964) (end 171.581854 36.943146) (width 1) (layer "B.Cu") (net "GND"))
 (segment (start 189.435 21.18) (end 190.685 21.18) (width 0.9) (layer "F.Cu") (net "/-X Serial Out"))
 (segment (start 186.506068 8.056068) (end 175.55 -2.9) (width 0.9) (layer "F.Cu") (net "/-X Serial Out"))
 (segment (start 189.435 21.18) (end 189.435 15.127136) (width 0.9) (layer "F.Cu") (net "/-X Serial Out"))
 (arc (start 186.506068 8.056068) (mid 188.673796 11.300302) (end 189.435 15.127136) (width 0.9) (layer "F.Cu") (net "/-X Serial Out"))
 (segment (start 174.3 -2.9) (end 167.428932 3.971068) (width 1) (layer "F.Cu") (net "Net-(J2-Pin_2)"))
 (segment (start 167.428932 142.528932) (end 174.364214 149.464214) (width 1) (layer "F.Cu") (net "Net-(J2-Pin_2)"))
 (segment (start 174.95 150.878427) (end 174.95 151.1) (width 1) (layer "F.Cu") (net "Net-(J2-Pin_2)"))
 (segment (start 164.5 11.042136) (end 164.5 135.457864) (width 1) (layer "F.Cu") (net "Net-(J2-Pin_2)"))
 (arc (start 174.95 150.878427) (mid 174.797759 150.11306) (end 174.364214 149.464214) (width 1) (layer "F.Cu") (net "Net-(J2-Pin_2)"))
 (arc (start 164.5 11.042136) (mid 165.261205 7.215302) (end 167.428932 3.971068) (width 1) (layer "F.Cu") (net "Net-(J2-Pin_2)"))
 (arc (start 164.5 135.457864) (mid 165.261204 139.284698) (end 167.428932 142.528932) (width 1) (layer "F.Cu") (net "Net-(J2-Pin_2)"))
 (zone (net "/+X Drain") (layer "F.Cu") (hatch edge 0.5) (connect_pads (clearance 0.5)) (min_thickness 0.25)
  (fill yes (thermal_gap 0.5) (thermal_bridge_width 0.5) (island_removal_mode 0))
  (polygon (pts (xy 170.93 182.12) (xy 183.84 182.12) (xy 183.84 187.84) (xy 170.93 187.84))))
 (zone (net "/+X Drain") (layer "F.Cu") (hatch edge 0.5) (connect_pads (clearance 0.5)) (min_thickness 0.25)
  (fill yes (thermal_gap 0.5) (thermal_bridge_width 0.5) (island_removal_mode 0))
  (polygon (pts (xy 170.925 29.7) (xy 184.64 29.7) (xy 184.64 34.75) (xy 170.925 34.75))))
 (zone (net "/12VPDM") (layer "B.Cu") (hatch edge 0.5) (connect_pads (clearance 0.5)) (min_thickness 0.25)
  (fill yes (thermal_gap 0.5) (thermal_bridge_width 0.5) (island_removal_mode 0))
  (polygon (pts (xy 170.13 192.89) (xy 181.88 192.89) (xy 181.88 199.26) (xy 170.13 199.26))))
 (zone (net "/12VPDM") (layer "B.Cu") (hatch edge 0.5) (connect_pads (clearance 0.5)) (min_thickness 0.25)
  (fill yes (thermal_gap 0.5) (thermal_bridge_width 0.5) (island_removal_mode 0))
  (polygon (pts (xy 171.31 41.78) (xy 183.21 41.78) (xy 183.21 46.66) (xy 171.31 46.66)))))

